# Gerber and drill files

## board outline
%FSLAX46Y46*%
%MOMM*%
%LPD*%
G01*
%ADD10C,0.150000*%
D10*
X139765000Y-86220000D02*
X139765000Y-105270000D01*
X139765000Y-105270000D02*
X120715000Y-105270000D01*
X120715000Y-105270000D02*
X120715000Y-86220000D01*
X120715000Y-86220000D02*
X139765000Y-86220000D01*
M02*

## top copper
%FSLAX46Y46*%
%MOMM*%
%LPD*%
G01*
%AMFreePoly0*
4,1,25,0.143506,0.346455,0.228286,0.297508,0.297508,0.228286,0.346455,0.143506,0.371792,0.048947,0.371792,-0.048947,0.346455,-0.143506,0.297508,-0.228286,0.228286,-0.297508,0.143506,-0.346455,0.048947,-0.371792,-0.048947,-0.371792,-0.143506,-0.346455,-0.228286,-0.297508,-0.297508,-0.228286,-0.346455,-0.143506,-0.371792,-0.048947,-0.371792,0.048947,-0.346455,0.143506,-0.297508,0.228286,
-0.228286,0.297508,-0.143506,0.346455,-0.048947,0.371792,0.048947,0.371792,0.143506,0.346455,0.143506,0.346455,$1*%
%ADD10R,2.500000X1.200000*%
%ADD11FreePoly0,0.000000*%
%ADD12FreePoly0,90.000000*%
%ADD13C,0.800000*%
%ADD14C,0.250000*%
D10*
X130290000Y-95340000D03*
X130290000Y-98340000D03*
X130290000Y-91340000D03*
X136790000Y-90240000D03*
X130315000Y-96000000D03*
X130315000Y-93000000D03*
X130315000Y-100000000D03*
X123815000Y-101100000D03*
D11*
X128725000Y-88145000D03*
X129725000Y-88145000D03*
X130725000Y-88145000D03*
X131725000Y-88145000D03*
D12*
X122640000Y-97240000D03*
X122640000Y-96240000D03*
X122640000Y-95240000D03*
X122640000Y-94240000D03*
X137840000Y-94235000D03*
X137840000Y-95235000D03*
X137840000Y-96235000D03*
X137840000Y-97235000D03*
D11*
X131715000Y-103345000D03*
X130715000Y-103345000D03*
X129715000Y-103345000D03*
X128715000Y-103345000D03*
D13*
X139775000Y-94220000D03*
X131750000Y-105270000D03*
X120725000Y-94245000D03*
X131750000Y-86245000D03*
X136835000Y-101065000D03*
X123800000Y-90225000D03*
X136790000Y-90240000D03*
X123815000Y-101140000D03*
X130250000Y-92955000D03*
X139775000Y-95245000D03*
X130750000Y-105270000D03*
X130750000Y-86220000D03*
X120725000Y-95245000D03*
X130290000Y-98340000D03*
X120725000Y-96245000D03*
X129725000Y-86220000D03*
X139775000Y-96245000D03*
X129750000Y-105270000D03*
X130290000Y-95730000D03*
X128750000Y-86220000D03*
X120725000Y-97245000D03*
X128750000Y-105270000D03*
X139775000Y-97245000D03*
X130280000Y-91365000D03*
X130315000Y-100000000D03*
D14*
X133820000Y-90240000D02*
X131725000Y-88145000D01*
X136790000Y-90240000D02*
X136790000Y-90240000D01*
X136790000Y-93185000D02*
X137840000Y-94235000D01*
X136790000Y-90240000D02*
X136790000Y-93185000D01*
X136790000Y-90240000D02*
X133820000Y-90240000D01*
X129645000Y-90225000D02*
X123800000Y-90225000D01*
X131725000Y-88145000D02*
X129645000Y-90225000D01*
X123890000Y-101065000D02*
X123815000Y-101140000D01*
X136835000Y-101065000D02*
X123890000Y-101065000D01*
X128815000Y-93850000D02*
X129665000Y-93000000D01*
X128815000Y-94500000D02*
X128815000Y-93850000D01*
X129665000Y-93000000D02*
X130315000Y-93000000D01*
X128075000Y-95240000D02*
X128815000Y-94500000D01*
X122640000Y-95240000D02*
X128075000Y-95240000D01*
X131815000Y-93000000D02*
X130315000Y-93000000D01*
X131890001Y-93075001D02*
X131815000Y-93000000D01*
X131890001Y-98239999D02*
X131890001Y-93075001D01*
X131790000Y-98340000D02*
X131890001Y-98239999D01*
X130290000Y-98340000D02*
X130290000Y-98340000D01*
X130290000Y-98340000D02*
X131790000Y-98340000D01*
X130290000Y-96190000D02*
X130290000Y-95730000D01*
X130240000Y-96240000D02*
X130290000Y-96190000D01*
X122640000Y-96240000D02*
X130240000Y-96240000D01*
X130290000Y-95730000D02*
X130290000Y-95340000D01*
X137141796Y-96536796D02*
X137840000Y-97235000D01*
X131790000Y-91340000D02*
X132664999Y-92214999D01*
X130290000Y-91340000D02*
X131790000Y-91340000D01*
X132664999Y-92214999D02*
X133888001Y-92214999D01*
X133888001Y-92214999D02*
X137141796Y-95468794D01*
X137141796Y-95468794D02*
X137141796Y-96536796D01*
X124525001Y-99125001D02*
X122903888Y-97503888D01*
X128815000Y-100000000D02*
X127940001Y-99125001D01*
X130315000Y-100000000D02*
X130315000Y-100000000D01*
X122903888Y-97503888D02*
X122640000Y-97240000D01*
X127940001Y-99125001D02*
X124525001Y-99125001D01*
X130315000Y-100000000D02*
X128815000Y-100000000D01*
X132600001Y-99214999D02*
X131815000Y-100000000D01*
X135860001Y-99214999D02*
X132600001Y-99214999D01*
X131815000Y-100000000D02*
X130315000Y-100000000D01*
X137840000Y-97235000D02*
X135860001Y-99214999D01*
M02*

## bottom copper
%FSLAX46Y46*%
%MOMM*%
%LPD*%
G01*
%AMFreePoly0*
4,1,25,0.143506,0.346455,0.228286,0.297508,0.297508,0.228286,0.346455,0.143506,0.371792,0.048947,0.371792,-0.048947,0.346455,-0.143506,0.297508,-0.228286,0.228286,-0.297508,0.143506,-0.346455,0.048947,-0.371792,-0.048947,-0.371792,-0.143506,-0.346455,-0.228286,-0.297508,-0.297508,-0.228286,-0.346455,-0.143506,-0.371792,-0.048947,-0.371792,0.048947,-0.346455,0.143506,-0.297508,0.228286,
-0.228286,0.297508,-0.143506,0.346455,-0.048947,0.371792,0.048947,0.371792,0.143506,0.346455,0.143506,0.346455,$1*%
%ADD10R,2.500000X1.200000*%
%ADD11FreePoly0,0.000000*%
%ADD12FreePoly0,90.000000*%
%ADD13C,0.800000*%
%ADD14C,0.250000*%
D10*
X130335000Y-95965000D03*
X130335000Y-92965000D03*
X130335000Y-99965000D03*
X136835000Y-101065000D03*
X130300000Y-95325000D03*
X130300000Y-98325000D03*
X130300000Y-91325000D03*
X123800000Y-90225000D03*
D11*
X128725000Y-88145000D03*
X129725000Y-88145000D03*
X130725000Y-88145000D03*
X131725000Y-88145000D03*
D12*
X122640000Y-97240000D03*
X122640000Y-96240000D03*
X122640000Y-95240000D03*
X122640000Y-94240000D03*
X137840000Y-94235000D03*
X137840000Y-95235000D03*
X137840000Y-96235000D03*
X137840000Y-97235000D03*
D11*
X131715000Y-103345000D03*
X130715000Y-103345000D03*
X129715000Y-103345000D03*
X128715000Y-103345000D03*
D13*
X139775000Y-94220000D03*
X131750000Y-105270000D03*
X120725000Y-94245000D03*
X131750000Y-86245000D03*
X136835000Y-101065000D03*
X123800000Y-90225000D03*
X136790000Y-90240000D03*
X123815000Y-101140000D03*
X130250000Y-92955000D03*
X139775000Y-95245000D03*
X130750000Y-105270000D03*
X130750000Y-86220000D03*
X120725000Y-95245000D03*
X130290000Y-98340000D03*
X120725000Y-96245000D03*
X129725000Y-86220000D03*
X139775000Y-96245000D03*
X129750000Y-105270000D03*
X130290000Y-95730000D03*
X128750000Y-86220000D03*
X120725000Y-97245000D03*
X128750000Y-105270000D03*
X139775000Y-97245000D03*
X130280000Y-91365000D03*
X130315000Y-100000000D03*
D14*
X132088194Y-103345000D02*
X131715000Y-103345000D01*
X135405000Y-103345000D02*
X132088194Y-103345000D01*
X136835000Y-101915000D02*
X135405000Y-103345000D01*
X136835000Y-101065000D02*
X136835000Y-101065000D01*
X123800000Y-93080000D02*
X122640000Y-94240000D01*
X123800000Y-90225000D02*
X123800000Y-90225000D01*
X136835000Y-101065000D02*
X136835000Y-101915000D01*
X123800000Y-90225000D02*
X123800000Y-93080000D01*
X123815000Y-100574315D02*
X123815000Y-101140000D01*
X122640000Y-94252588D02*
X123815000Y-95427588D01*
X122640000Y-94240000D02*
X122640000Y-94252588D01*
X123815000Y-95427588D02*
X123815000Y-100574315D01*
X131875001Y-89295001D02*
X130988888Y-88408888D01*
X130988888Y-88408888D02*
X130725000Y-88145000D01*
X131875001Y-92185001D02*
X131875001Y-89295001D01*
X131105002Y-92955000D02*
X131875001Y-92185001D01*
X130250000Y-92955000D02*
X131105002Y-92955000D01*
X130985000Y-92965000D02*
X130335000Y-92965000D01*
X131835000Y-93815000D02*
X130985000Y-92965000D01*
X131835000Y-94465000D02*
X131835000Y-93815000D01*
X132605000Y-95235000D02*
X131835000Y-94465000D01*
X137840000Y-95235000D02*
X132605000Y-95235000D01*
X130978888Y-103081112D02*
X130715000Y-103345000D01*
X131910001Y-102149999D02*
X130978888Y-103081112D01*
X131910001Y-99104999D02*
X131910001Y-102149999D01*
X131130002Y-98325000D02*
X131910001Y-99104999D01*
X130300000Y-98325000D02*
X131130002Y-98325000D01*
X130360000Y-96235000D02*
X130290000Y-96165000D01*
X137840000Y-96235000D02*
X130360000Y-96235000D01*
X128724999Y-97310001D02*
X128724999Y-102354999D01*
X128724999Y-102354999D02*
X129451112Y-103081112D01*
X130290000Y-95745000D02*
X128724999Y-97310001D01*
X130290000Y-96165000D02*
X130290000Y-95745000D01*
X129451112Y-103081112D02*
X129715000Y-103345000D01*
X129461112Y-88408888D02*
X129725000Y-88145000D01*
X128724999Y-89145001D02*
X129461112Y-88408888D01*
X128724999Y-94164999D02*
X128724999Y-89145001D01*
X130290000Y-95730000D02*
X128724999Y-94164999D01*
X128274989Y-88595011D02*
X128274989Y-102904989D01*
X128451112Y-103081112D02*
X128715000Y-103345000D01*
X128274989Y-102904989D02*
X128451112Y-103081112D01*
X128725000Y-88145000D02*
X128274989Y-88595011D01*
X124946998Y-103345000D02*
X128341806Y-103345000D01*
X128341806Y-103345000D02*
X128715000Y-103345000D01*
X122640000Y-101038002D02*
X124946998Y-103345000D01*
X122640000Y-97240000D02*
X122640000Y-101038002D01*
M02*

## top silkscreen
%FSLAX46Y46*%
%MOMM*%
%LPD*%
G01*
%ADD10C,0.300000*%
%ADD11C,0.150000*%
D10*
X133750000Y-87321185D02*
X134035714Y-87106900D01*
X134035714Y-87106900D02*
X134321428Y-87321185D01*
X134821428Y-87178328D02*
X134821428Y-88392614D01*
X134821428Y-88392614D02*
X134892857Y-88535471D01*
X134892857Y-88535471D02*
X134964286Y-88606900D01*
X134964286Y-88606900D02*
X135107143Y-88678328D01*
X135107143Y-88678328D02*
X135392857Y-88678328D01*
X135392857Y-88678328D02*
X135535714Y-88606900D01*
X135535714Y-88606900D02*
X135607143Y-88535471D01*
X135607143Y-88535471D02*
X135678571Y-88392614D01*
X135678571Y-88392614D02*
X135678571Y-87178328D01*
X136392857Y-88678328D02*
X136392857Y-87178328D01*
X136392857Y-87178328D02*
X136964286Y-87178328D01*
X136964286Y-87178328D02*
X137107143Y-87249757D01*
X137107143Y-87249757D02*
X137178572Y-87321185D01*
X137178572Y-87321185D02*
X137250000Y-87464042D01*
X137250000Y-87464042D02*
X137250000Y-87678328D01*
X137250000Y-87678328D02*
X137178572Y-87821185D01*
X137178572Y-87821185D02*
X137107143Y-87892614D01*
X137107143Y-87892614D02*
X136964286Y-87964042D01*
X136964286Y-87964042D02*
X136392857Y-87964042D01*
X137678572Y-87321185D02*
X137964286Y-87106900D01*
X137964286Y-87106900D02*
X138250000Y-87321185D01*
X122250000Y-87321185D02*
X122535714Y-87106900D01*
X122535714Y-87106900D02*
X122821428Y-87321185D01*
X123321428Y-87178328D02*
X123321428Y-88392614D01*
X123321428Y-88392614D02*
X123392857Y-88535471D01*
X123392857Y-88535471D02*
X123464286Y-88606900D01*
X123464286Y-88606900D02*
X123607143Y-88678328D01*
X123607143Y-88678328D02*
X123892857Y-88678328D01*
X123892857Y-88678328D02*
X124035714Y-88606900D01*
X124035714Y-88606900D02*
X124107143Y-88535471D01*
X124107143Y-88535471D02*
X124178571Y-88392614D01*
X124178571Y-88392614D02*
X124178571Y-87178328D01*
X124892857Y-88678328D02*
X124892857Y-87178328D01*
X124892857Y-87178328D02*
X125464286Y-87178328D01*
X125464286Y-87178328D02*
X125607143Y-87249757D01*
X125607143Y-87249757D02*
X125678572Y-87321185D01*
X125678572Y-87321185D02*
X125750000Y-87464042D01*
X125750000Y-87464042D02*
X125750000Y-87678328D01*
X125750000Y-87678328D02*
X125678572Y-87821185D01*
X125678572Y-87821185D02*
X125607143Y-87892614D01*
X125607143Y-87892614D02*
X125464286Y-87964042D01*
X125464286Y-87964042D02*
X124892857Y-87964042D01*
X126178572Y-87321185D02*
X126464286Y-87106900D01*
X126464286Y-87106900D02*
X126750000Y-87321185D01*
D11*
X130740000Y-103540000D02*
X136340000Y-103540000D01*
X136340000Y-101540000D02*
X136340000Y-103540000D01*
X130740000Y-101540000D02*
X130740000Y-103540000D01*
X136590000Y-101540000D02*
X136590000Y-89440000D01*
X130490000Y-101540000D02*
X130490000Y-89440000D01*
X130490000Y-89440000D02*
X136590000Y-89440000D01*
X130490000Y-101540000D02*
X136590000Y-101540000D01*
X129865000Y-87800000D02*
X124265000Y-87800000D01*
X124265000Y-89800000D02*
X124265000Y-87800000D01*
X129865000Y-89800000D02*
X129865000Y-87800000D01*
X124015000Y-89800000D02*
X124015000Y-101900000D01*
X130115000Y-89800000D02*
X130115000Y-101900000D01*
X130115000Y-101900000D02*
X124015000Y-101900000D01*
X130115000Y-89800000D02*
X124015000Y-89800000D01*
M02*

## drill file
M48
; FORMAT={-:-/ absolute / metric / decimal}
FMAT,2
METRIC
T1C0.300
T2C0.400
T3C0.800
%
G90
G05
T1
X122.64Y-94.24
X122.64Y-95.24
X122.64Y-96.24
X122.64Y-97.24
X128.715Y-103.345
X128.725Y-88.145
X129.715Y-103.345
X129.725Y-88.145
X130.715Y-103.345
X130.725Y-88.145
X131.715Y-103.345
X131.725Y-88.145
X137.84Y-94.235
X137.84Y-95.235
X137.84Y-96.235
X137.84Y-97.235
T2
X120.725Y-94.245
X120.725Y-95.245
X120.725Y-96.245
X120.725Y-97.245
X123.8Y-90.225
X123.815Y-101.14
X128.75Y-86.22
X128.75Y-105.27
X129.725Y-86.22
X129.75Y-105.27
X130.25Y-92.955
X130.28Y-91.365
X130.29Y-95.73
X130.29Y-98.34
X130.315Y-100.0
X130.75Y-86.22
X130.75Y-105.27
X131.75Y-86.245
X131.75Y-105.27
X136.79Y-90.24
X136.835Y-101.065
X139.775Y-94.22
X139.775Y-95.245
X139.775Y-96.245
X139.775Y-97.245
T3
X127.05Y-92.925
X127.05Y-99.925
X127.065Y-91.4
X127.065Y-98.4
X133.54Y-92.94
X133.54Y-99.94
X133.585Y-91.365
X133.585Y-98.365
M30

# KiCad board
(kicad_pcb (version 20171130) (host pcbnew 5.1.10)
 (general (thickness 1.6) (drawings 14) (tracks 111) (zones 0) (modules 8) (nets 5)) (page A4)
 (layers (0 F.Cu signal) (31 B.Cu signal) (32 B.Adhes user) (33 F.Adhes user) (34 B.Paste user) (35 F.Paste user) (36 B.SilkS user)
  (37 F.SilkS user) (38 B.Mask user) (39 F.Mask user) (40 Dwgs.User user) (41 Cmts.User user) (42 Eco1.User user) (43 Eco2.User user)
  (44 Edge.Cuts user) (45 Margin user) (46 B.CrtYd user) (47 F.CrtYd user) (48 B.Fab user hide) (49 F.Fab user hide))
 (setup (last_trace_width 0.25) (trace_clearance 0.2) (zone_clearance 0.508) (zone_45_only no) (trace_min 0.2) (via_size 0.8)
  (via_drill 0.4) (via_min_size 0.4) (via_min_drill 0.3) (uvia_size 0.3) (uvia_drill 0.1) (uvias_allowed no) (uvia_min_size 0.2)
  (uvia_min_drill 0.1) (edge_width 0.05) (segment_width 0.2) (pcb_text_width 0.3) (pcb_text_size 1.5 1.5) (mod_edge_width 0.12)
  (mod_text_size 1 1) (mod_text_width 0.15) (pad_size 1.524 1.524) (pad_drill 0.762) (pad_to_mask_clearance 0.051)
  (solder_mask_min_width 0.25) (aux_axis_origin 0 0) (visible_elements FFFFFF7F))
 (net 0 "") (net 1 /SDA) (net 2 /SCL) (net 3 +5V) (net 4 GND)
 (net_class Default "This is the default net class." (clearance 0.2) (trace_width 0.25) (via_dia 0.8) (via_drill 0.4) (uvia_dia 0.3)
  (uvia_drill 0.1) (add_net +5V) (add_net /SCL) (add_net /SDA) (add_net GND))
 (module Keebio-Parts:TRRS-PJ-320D (layer B.Cu) (at 133.585 89.765 180)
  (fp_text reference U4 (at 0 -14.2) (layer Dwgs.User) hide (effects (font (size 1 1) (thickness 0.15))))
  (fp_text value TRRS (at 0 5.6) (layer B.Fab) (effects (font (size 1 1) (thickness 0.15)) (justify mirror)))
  (pad 3 smd rect (at 3.25 -6.2 180) (size 2.5 1.2) (layers B.Cu B.Paste B.Mask) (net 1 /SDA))
  (pad "" np_thru_hole circle (at 0 -1.6 180) (size 0.8 0.8) (drill 0.8) (layers *.Cu *.Mask))
  (pad "" np_thru_hole circle (at 0 -8.6 180) (size 0.8 0.8) (drill 0.8) (layers *.Cu *.Mask))
  (pad 4 smd rect (at 3.25 -3.2 180) (size 2.5 1.2) (layers B.Cu B.Paste B.Mask) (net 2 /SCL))
  (pad 2 smd rect (at 3.25 -10.2 180) (size 2.5 1.2) (layers B.Cu B.Paste B.Mask) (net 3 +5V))
  (pad 1 smd rect (at -3.25 -11.3 180) (size 2.5 1.2) (layers B.Cu B.Paste B.Mask) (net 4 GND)))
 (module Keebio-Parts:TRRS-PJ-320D (layer F.Cu) (at 133.54 101.54 180)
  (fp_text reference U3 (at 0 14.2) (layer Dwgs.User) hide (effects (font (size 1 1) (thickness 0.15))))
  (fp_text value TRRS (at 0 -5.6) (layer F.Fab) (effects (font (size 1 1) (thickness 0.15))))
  (fp_line (start 2.8 -2) (end -2.8 -2) (layer F.SilkS) (width 0.15))
  (fp_line (start -2.8 0) (end -2.8 -2) (layer F.SilkS) (width 0.15))
  (fp_line (start 2.8 0) (end 2.8 -2) (layer F.SilkS) (width 0.15))
  (fp_line (start -3.05 0) (end -3.05 12.1) (layer F.SilkS) (width 0.15))
  (fp_line (start 3.05 0) (end 3.05 12.1) (layer F.SilkS) (width 0.15))
  (fp_line (start 3.05 12.1) (end -3.05 12.1) (layer F.SilkS) (width 0.15))
  (fp_line (start 3.05 0) (end -3.05 0) (layer F.SilkS) (width 0.15))
  (pad 3 smd rect (at 3.25 6.2 180) (size 2.5 1.2) (layers F.Cu F.Paste F.Mask) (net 1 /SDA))
  (pad "" np_thru_hole circle (at 0 1.6 180) (size 0.8 0.8) (drill 0.8) (layers *.Cu *.Mask))
  (pad "" np_thru_hole circle (at 0 8.6 180) (size 0.8 0.8) (drill 0.8) (layers *.Cu *.Mask))
  (pad 4 smd rect (at 3.25 3.2 180) (size 2.5 1.2) (layers F.Cu F.Paste F.Mask) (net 2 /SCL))
  (pad 2 smd rect (at 3.25 10.2 180) (size 2.5 1.2) (layers F.Cu F.Paste F.Mask) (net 3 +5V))
  (pad 1 smd rect (at -3.25 11.3 180) (size 2.5 1.2) (layers F.Cu F.Paste F.Mask) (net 4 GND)))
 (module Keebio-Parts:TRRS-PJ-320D (layer F.Cu) (at 127.065 89.8)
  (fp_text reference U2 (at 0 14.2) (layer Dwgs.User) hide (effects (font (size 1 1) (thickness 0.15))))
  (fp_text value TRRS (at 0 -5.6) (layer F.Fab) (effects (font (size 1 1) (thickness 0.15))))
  (fp_line (start 2.8 -2) (end -2.8 -2) (layer F.SilkS) (width 0.15))
  (fp_line (start -2.8 0) (end -2.8 -2) (layer F.SilkS) (width 0.15))
  (fp_line (start 2.8 0) (end 2.8 -2) (layer F.SilkS) (width 0.15))
  (fp_line (start -3.05 0) (end -3.05 12.1) (layer F.SilkS) (width 0.15))
  (fp_line (start 3.05 0) (end 3.05 12.1) (layer F.SilkS) (width 0.15))
  (fp_line (start 3.05 12.1) (end -3.05 12.1) (layer F.SilkS) (width 0.15))
  (fp_line (start 3.05 0) (end -3.05 0) (layer F.SilkS) (width 0.15))
  (pad 3 smd rect (at 3.25 6.2) (size 2.5 1.2) (layers F.Cu F.Paste F.Mask) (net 1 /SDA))
  (pad "" np_thru_hole circle (at 0 1.6) (size 0.8 0.8) (drill 0.8) (layers *.Cu *.Mask))
  (pad "" np_thru_hole circle (at 0 8.6) (size 0.8 0.8) (drill 0.8) (layers *.Cu *.Mask))
  (pad 4 smd rect (at 3.25 3.2) (size 2.5 1.2) (layers F.Cu F.Paste F.Mask) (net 2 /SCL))
  (pad 2 smd rect (at 3.25 10.2) (size 2.5 1.2) (layers F.Cu F.Paste F.Mask) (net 3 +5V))
  (pad 1 smd rect (at -3.25 11.3) (size 2.5 1.2) (layers F.Cu F.Paste F.Mask) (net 4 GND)))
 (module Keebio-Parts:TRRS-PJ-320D (layer B.Cu) (at 127.05 101.525)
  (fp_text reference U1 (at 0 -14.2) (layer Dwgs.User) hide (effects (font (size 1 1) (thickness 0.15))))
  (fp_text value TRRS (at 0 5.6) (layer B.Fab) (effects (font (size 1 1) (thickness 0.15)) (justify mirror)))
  (pad 3 smd rect (at 3.25 -6.2) (size 2.5 1.2) (layers B.Cu B.Paste B.Mask) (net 1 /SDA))
  (pad "" np_thru_hole circle (at 0 -1.6) (size 0.8 0.8) (drill 0.8) (layers *.Cu *.Mask))
  (pad "" np_thru_hole circle (at 0 -8.6) (size 0.8 0.8) (drill 0.8) (layers *.Cu *.Mask))
  (pad 4 smd rect (at 3.25 -3.2) (size 2.5 1.2) (layers B.Cu B.Paste B.Mask) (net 2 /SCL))
  (pad 2 smd rect (at 3.25 -10.2) (size 2.5 1.2) (layers B.Cu B.Paste B.Mask) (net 3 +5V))
  (pad 1 smd rect (at -3.25 -11.3) (size 2.5 1.2) (layers B.Cu B.Paste B.Mask) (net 4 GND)))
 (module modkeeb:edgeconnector (layer B.Cu) (at 130.225 86.145)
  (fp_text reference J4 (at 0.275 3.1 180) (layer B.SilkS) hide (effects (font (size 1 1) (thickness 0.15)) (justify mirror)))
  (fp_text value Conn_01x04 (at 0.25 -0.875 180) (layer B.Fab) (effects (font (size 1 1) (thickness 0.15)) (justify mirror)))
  (pad 1 thru_hole custom (at -1.5 2) (size 0.75 0.75) (drill 0.3) (layers *.Cu *.Mask) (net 3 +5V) (zone_connect 0)
   (options (clearance outline) (anchor circle)) (primitives))
  (pad 2 thru_hole custom (at -0.5 2) (size 0.75 0.75) (drill 0.3) (layers *.Cu *.Mask) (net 1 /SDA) (zone_connect 0)
   (options (clearance outline) (anchor circle)) (primitives))
  (pad 3 thru_hole custom (at 0.5 2) (size 0.75 0.75) (drill 0.3) (layers *.Cu *.Mask) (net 2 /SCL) (zone_connect 0)
   (options (clearance outline) (anchor circle)) (primitives))
  (pad 4 thru_hole custom (at 1.5 2) (size 0.75 0.75) (drill 0.3) (layers *.Cu *.Mask) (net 4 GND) (zone_connect 0)
   (options (clearance outline) (anchor circle)) (primitives)))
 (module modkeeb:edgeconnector (layer B.Cu) (at 120.64 95.74 90)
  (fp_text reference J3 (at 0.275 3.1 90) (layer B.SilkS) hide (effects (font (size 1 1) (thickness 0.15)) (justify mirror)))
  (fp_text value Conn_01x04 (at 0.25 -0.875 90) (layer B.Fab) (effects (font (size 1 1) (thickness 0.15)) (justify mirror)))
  (pad 1 thru_hole custom (at -1.5 2 90) (size 0.75 0.75) (drill 0.3) (layers *.Cu *.Mask) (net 3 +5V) (zone_connect 0)
   (options (clearance outline) (anchor circle)) (primitives))
  (pad 2 thru_hole custom (at -0.5 2 90) (size 0.75 0.75) (drill 0.3) (layers *.Cu *.Mask) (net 1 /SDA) (zone_connect 0)
   (options (clearance outline) (anchor circle)) (primitives))
  (pad 3 thru_hole custom (at 0.5 2 90) (size 0.75 0.75) (drill 0.3) (layers *.Cu *.Mask) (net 2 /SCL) (zone_connect 0)
   (options (clearance outline) (anchor circle)) (primitives))
  (pad 4 thru_hole custom (at 1.5 2 90) (size 0.75 0.75) (drill 0.3) (layers *.Cu *.Mask) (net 4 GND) (zone_connect 0)
   (options (clearance outline) (anchor circle)) (primitives)))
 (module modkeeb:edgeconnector (layer F.Cu) (at 139.84 95.735 90)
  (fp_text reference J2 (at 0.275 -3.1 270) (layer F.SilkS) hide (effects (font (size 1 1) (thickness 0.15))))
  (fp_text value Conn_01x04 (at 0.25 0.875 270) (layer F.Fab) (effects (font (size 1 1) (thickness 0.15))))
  (pad 4 thru_hole custom (at 1.5 -2 90) (size 0.75 0.75) (drill 0.3) (layers *.Cu *.Mask) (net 4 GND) (zone_connect 0)
   (options (clearance outline) (anchor circle)) (primitives))
  (pad 3 thru_hole custom (at 0.5 -2 90) (size 0.75 0.75) (drill 0.3) (layers *.Cu *.Mask) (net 2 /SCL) (zone_connect 0)
   (options (clearance outline) (anchor circle)) (primitives))
  (pad 2 thru_hole custom (at -0.5 -2 90) (size 0.75 0.75) (drill 0.3) (layers *.Cu *.Mask) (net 1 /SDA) (zone_connect 0)
   (options (clearance outline) (anchor circle)) (primitives))
  (pad 1 thru_hole custom (at -1.5 -2 90) (size 0.75 0.75) (drill 0.3) (layers *.Cu *.Mask) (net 3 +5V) (zone_connect 0)
   (options (clearance outline) (anchor circle)) (primitives)))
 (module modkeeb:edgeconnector (layer F.Cu) (at 130.215 105.345)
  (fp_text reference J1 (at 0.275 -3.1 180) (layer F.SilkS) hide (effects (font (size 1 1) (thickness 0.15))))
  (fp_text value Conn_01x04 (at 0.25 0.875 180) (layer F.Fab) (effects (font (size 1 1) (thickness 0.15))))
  (pad 4 thru_hole custom (at 1.5 -2) (size 0.75 0.75) (drill 0.3) (layers *.Cu *.Mask) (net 4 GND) (zone_connect 0)
   (options (clearance outline) (anchor circle)) (primitives))
  (pad 3 thru_hole custom (at 0.5 -2) (size 0.75 0.75) (drill 0.3) (layers *.Cu *.Mask) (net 2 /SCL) (zone_connect 0)
   (options (clearance outline) (anchor circle)) (primitives))
  (pad 2 thru_hole custom (at -0.5 -2) (size 0.75 0.75) (drill 0.3) (layers *.Cu *.Mask) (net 1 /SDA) (zone_connect 0)
   (options (clearance outline) (anchor circle)) (primitives))
  (pad 1 thru_hole custom (at -1.5 -2) (size 0.75 0.75) (drill 0.3) (layers *.Cu *.Mask) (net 3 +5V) (zone_connect 0)
   (options (clearance outline) (anchor circle)) (primitives)))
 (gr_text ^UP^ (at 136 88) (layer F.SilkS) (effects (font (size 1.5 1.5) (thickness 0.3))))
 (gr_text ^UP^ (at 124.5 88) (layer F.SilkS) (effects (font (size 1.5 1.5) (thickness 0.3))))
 (gr_line (start 139.765 86.22) (end 139.765 105.27) (layer Edge.Cuts) (width 0.15))
 (gr_line (start 139.765 105.27) (end 120.715 105.27) (layer Edge.Cuts) (width 0.15))
 (gr_line (start 120.715 105.27) (end 120.715 86.22) (layer Edge.Cuts) (width 0.15))
 (gr_line (start 120.715 86.22) (end 139.765 86.22) (layer Edge.Cuts) (width 0.15))
 (via (at 139.775 94.22) (size 0.8) (drill 0.4) (layers F.Cu B.Cu) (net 4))
 (via (at 131.75 105.27) (size 0.8) (drill 0.4) (layers F.Cu B.Cu) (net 4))
 (via (at 120.725 94.245) (size 0.8) (drill 0.4) (layers F.Cu B.Cu) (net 4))
 (via (at 131.75 86.245) (size 0.8) (drill 0.4) (layers F.Cu B.Cu) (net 4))
 (segment (start 132.088194 103.345) (end 131.715 103.345) (width 0.25) (layer B.Cu) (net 4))
 (segment (start 135.405 103.345) (end 132.088194 103.345) (width 0.25) (layer B.Cu) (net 4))
 (segment (start 136.835 101.915) (end 135.405 103.345) (width 0.25) (layer B.Cu) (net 4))
 (segment (start 136.835 101.065) (end 136.835 101.065) (width 0.25) (layer B.Cu) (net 4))
 (segment (start 123.8 93.08) (end 122.64 94.24) (width 0.25) (layer B.Cu) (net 4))
 (segment (start 123.8 90.225) (end 123.8 90.225) (width 0.25) (layer B.Cu) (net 4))
 (segment (start 133.82 90.24) (end 131.725 88.145) (width 0.25) (layer F.Cu) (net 4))
 (segment (start 136.79 90.24) (end 136.79 90.24) (width 0.25) (layer F.Cu) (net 4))
 (segment (start 136.79 93.185) (end 137.84 94.235) (width 0.25) (layer F.Cu) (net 4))
 (segment (start 136.79 90.24) (end 136.79 93.185) (width 0.25) (layer F.Cu) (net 4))
 (segment (start 136.835 101.065) (end 136.835 101.915) (width 0.25) (layer B.Cu) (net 4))
 (via (at 136.835 101.065) (size 0.8) (drill 0.4) (layers F.Cu B.Cu) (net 4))
 (segment (start 123.8 90.225) (end 123.8 93.08) (width 0.25) (layer B.Cu) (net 4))
 (via (at 123.8 90.225) (size 0.8) (drill 0.4) (layers F.Cu B.Cu) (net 4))
 (segment (start 136.79 90.24) (end 133.82 90.24) (width 0.25) (layer F.Cu) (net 4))
 (via (at 136.79 90.24) (size 0.8) (drill 0.4) (layers F.Cu B.Cu) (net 4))
 (segment (start 123.815 100.574315) (end 123.815 101.14) (width 0.25) (layer B.Cu) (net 4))
 (segment (start 122.64 94.252588) (end 123.815 95.427588) (width 0.25) (layer B.Cu) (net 4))
 (segment (start 122.64 94.24) (end 122.64 94.252588) (width 0.25) (layer B.Cu) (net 4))
 (segment (start 123.815 95.427588) (end 123.815 100.574315) (width 0.25) (layer B.Cu) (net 4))
 (via (at 123.815 101.14) (size 0.8) (drill 0.4) (layers F.Cu B.Cu) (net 4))
 (segment (start 129.645 90.225) (end 123.8 90.225) (width 0.25) (layer F.Cu) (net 4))
 (segment (start 131.725 88.145) (end 129.645 90.225) (width 0.25) (layer F.Cu) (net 4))
 (segment (start 123.89 101.065) (end 123.815 101.14) (width 0.25) (layer F.Cu) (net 4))
 (segment (start 136.835 101.065) (end 123.89 101.065) (width 0.25) (layer F.Cu) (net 4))
 (via (at 130.25 92.955) (size 0.8) (drill 0.4) (layers F.Cu B.Cu) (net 2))
 (via (at 139.775 95.245) (size 0.8) (drill 0.4) (layers F.Cu B.Cu) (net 2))
 (via (at 130.75 105.27) (size 0.8) (drill 0.4) (layers F.Cu B.Cu) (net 2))
 (via (at 130.75 86.22) (size 0.8) (drill 0.4) (layers F.Cu B.Cu) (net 2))
 (via (at 120.725 95.245) (size 0.8) (drill 0.4) (layers F.Cu B.Cu) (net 2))
 (segment (start 131.875001 89.295001) (end 130.988888 88.408888) (width 0.25) (layer B.Cu) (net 2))
 (segment (start 130.988888 88.408888) (end 130.725 88.145) (width 0.25) (layer B.Cu) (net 2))
 (segment (start 131.875001 92.185001) (end 131.875001 89.295001) (width 0.25) (layer B.Cu) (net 2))
 (segment (start 131.105002 92.955) (end 131.875001 92.185001) (width 0.25) (layer B.Cu) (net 2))
 (segment (start 130.25 92.955) (end 131.105002 92.955) (width 0.25) (layer B.Cu) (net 2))
 (segment (start 130.985 92.965) (end 130.335 92.965) (width 0.25) (layer B.Cu) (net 2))
 (segment (start 131.835 93.815) (end 130.985 92.965) (width 0.25) (layer B.Cu) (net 2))
 (segment (start 131.835 94.465) (end 131.835 93.815) (width 0.25) (layer B.Cu) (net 2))
 (segment (start 132.605 95.235) (end 131.835 94.465) (width 0.25) (layer B.Cu) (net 2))
 (segment (start 137.84 95.235) (end 132.605 95.235) (width 0.25) (layer B.Cu) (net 2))
 (segment (start 128.815 93.85) (end 129.665 93) (width 0.25) (layer F.Cu) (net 2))
 (segment (start 128.815 94.5) (end 128.815 93.85) (width 0.25) (layer F.Cu) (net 2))
 (segment (start 129.665 93) (end 130.315 93) (width 0.25) (layer F.Cu) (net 2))
 (segment (start 128.075 95.24) (end 128.815 94.5) (width 0.25) (layer F.Cu) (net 2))
 (segment (start 122.64 95.24) (end 128.075 95.24) (width 0.25) (layer F.Cu) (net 2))
 (segment (start 131.815 93) (end 130.315 93) (width 0.25) (layer F.Cu) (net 2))
 (segment (start 131.890001 93.075001) (end 131.815 93) (width 0.25) (layer F.Cu) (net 2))
 (segment (start 131.890001 98.239999) (end 131.890001 93.075001) (width 0.25) (layer F.Cu) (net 2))
 (segment (start 131.79 98.34) (end 131.890001 98.239999) (width 0.25) (layer F.Cu) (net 2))
 (segment (start 130.29 98.34) (end 130.29 98.34) (width 0.25) (layer F.Cu) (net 2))
 (segment (start 130.29 98.34) (end 131.79 98.34) (width 0.25) (layer F.Cu) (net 2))
 (via (at 130.29 98.34) (size 0.8) (drill 0.4) (layers F.Cu B.Cu) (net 2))
 (segment (start 130.978888 103.081112) (end 130.715 103.345) (width 0.25) (layer B.Cu) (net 2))
 (segment (start 131.910001 102.149999) (end 130.978888 103.081112) (width 0.25) (layer B.Cu) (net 2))
 (segment (start 131.910001 99.104999) (end 131.910001 102.149999) (width 0.25) (layer B.Cu) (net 2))
 (segment (start 131.130002 98.325) (end 131.910001 99.104999) (width 0.25) (layer B.Cu) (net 2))
 (segment (start 130.3 98.325) (end 131.130002 98.325) (width 0.25) (layer B.Cu) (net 2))
 (via (at 120.725 96.245) (size 0.8) (drill 0.4) (layers F.Cu B.Cu) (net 1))
 (via (at 129.725 86.22) (size 0.8) (drill 0.4) (layers F.Cu B.Cu) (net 1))
 (via (at 139.775 96.245) (size 0.8) (drill 0.4) (layers F.Cu B.Cu) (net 1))
 (via (at 129.75 105.27) (size 0.8) (drill 0.4) (layers F.Cu B.Cu) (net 1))
 (segment (start 130.36 96.235) (end 130.29 96.165) (width 0.25) (layer B.Cu) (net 1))
 (segment (start 137.84 96.235) (end 130.36 96.235) (width 0.25) (layer B.Cu) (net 1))
 (segment (start 128.724999 97.310001) (end 128.724999 102.354999) (width 0.25) (layer B.Cu) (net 1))
 (segment (start 128.724999 102.354999) (end 129.451112 103.081112) (width 0.25) (layer B.Cu) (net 1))
 (segment (start 130.29 95.745) (end 128.724999 97.310001) (width 0.25) (layer B.Cu) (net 1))
 (segment (start 130.29 96.165) (end 130.29 95.745) (width 0.25) (layer B.Cu) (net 1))
 (segment (start 129.451112 103.081112) (end 129.715 103.345) (width 0.25) (layer B.Cu) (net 1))
 (segment (start 130.29 96.19) (end 130.29 95.73) (width 0.25) (layer F.Cu) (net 1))
 (segment (start 130.24 96.24) (end 130.29 96.19) (width 0.25) (layer F.Cu) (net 1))
 (segment (start 122.64 96.24) (end 130.24 96.24) (width 0.25) (layer F.Cu) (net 1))
 (segment (start 130.29 95.73) (end 130.29 95.34) (width 0.25) (layer F.Cu) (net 1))
 (via (at 130.29 95.73) (size 0.8) (drill 0.4) (layers F.Cu B.Cu) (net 1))
 (segment (start 129.461112 88.408888) (end 129.725 88.145) (width 0.25) (layer B.Cu) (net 1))
 (segment (start 128.724999 89.145001) (end 129.461112 88.408888) (width 0.25) (layer B.Cu) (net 1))
 (segment (start 128.724999 94.164999) (end 128.724999 89.145001) (width 0.25) (layer B.Cu) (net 1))
 (segment (start 130.29 95.73) (end 128.724999 94.164999) (width 0.25) (layer B.Cu) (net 1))
 (via (at 128.75 86.22) (size 0.8) (drill 0.4) (layers F.Cu B.Cu) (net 3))
 (via (at 120.725 97.245) (size 0.8) (drill 0.4) (layers F.Cu B.Cu) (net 3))
 (via (at 128.75 105.27) (size 0.8) (drill 0.4) (layers F.Cu B.Cu) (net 3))
 (via (at 139.775 97.245) (size 0.8) (drill 0.4) (layers F.Cu B.Cu) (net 3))
 (via (at 130.28 91.365) (size 0.8) (drill 0.4) (layers F.Cu B.Cu) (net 3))
 (segment (start 137.141796 96.536796) (end 137.84 97.235) (width 0.25) (layer F.Cu) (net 3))
 (segment (start 131.79 91.34) (end 132.664999 92.214999) (width 0.25) (layer F.Cu) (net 3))
 (segment (start 130.29 91.34) (end 131.79 91.34) (width 0.25) (layer F.Cu) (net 3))
 (segment (start 132.664999 92.214999) (end 133.888001 92.214999) (width 0.25) (layer F.Cu) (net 3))
 (segment (start 133.888001 92.214999) (end 137.141796 95.468794) (width 0.25) (layer F.Cu) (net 3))
 (segment (start 137.141796 95.468794) (end 137.141796 96.536796) (width 0.25) (layer F.Cu) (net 3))
 (segment (start 124.525001 99.125001) (end 122.903888 97.503888) (width 0.25) (layer F.Cu) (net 3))
 (segment (start 128.815 100) (end 127.940001 99.125001) (width 0.25) (layer F.Cu) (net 3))
 (segment (start 130.315 100) (end 130.315 100) (width 0.25) (layer F.Cu) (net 3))
 (segment (start 122.903888 97.503888) (end 122.64 97.24) (width 0.25) (layer F.Cu) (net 3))
 (segment (start 127.940001 99.125001) (end 124.525001 99.125001) (width 0.25) (layer F.Cu) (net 3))
 (segment (start 128.274989 88.595011) (end 128.274989 102.904989) (width 0.25) (layer B.Cu) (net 3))
 (segment (start 128.451112 103.081112) (end 128.715 103.345) (width 0.25) (layer B.Cu) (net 3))
 (segment (start 128.274989 102.904989) (end 128.451112 103.081112) (width 0.25) (layer B.Cu) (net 3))
 (segment (start 128.725 88.145) (end 128.274989 88.595011) (width 0.25) (layer B.Cu) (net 3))
 (segment (start 124.946998 103.345) (end 128.341806 103.345) (width 0.25) (layer B.Cu) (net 3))
 (segment (start 128.341806 103.345) (end 128.715 103.345) (width 0.25) (layer B.Cu) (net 3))
 (segment (start 122.64 101.038002) (end 124.946998 103.345) (width 0.25) (layer B.Cu) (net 3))
 (segment (start 122.64 97.24) (end 122.64 101.038002) (width 0.25) (layer B.Cu) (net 3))
 (segment (start 130.315 100) (end 128.815 100) (width 0.25) (layer F.Cu) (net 3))
 (via (at 130.315 100) (size 0.8) (drill 0.4) (layers F.Cu B.Cu) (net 3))
 (segment (start 132.600001 99.214999) (end 131.815 100) (width 0.25) (layer F.Cu) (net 3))
 (segment (start 135.860001 99.214999) (end 132.600001 99.214999) (width 0.25) (layer F.Cu) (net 3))
 (segment (start 131.815 100) (end 130.315 100) (width 0.25) (layer F.Cu) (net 3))
 (segment (start 137.84 97.235) (end 135.860001 99.214999) (width 0.25) (layer F.Cu) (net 3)))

